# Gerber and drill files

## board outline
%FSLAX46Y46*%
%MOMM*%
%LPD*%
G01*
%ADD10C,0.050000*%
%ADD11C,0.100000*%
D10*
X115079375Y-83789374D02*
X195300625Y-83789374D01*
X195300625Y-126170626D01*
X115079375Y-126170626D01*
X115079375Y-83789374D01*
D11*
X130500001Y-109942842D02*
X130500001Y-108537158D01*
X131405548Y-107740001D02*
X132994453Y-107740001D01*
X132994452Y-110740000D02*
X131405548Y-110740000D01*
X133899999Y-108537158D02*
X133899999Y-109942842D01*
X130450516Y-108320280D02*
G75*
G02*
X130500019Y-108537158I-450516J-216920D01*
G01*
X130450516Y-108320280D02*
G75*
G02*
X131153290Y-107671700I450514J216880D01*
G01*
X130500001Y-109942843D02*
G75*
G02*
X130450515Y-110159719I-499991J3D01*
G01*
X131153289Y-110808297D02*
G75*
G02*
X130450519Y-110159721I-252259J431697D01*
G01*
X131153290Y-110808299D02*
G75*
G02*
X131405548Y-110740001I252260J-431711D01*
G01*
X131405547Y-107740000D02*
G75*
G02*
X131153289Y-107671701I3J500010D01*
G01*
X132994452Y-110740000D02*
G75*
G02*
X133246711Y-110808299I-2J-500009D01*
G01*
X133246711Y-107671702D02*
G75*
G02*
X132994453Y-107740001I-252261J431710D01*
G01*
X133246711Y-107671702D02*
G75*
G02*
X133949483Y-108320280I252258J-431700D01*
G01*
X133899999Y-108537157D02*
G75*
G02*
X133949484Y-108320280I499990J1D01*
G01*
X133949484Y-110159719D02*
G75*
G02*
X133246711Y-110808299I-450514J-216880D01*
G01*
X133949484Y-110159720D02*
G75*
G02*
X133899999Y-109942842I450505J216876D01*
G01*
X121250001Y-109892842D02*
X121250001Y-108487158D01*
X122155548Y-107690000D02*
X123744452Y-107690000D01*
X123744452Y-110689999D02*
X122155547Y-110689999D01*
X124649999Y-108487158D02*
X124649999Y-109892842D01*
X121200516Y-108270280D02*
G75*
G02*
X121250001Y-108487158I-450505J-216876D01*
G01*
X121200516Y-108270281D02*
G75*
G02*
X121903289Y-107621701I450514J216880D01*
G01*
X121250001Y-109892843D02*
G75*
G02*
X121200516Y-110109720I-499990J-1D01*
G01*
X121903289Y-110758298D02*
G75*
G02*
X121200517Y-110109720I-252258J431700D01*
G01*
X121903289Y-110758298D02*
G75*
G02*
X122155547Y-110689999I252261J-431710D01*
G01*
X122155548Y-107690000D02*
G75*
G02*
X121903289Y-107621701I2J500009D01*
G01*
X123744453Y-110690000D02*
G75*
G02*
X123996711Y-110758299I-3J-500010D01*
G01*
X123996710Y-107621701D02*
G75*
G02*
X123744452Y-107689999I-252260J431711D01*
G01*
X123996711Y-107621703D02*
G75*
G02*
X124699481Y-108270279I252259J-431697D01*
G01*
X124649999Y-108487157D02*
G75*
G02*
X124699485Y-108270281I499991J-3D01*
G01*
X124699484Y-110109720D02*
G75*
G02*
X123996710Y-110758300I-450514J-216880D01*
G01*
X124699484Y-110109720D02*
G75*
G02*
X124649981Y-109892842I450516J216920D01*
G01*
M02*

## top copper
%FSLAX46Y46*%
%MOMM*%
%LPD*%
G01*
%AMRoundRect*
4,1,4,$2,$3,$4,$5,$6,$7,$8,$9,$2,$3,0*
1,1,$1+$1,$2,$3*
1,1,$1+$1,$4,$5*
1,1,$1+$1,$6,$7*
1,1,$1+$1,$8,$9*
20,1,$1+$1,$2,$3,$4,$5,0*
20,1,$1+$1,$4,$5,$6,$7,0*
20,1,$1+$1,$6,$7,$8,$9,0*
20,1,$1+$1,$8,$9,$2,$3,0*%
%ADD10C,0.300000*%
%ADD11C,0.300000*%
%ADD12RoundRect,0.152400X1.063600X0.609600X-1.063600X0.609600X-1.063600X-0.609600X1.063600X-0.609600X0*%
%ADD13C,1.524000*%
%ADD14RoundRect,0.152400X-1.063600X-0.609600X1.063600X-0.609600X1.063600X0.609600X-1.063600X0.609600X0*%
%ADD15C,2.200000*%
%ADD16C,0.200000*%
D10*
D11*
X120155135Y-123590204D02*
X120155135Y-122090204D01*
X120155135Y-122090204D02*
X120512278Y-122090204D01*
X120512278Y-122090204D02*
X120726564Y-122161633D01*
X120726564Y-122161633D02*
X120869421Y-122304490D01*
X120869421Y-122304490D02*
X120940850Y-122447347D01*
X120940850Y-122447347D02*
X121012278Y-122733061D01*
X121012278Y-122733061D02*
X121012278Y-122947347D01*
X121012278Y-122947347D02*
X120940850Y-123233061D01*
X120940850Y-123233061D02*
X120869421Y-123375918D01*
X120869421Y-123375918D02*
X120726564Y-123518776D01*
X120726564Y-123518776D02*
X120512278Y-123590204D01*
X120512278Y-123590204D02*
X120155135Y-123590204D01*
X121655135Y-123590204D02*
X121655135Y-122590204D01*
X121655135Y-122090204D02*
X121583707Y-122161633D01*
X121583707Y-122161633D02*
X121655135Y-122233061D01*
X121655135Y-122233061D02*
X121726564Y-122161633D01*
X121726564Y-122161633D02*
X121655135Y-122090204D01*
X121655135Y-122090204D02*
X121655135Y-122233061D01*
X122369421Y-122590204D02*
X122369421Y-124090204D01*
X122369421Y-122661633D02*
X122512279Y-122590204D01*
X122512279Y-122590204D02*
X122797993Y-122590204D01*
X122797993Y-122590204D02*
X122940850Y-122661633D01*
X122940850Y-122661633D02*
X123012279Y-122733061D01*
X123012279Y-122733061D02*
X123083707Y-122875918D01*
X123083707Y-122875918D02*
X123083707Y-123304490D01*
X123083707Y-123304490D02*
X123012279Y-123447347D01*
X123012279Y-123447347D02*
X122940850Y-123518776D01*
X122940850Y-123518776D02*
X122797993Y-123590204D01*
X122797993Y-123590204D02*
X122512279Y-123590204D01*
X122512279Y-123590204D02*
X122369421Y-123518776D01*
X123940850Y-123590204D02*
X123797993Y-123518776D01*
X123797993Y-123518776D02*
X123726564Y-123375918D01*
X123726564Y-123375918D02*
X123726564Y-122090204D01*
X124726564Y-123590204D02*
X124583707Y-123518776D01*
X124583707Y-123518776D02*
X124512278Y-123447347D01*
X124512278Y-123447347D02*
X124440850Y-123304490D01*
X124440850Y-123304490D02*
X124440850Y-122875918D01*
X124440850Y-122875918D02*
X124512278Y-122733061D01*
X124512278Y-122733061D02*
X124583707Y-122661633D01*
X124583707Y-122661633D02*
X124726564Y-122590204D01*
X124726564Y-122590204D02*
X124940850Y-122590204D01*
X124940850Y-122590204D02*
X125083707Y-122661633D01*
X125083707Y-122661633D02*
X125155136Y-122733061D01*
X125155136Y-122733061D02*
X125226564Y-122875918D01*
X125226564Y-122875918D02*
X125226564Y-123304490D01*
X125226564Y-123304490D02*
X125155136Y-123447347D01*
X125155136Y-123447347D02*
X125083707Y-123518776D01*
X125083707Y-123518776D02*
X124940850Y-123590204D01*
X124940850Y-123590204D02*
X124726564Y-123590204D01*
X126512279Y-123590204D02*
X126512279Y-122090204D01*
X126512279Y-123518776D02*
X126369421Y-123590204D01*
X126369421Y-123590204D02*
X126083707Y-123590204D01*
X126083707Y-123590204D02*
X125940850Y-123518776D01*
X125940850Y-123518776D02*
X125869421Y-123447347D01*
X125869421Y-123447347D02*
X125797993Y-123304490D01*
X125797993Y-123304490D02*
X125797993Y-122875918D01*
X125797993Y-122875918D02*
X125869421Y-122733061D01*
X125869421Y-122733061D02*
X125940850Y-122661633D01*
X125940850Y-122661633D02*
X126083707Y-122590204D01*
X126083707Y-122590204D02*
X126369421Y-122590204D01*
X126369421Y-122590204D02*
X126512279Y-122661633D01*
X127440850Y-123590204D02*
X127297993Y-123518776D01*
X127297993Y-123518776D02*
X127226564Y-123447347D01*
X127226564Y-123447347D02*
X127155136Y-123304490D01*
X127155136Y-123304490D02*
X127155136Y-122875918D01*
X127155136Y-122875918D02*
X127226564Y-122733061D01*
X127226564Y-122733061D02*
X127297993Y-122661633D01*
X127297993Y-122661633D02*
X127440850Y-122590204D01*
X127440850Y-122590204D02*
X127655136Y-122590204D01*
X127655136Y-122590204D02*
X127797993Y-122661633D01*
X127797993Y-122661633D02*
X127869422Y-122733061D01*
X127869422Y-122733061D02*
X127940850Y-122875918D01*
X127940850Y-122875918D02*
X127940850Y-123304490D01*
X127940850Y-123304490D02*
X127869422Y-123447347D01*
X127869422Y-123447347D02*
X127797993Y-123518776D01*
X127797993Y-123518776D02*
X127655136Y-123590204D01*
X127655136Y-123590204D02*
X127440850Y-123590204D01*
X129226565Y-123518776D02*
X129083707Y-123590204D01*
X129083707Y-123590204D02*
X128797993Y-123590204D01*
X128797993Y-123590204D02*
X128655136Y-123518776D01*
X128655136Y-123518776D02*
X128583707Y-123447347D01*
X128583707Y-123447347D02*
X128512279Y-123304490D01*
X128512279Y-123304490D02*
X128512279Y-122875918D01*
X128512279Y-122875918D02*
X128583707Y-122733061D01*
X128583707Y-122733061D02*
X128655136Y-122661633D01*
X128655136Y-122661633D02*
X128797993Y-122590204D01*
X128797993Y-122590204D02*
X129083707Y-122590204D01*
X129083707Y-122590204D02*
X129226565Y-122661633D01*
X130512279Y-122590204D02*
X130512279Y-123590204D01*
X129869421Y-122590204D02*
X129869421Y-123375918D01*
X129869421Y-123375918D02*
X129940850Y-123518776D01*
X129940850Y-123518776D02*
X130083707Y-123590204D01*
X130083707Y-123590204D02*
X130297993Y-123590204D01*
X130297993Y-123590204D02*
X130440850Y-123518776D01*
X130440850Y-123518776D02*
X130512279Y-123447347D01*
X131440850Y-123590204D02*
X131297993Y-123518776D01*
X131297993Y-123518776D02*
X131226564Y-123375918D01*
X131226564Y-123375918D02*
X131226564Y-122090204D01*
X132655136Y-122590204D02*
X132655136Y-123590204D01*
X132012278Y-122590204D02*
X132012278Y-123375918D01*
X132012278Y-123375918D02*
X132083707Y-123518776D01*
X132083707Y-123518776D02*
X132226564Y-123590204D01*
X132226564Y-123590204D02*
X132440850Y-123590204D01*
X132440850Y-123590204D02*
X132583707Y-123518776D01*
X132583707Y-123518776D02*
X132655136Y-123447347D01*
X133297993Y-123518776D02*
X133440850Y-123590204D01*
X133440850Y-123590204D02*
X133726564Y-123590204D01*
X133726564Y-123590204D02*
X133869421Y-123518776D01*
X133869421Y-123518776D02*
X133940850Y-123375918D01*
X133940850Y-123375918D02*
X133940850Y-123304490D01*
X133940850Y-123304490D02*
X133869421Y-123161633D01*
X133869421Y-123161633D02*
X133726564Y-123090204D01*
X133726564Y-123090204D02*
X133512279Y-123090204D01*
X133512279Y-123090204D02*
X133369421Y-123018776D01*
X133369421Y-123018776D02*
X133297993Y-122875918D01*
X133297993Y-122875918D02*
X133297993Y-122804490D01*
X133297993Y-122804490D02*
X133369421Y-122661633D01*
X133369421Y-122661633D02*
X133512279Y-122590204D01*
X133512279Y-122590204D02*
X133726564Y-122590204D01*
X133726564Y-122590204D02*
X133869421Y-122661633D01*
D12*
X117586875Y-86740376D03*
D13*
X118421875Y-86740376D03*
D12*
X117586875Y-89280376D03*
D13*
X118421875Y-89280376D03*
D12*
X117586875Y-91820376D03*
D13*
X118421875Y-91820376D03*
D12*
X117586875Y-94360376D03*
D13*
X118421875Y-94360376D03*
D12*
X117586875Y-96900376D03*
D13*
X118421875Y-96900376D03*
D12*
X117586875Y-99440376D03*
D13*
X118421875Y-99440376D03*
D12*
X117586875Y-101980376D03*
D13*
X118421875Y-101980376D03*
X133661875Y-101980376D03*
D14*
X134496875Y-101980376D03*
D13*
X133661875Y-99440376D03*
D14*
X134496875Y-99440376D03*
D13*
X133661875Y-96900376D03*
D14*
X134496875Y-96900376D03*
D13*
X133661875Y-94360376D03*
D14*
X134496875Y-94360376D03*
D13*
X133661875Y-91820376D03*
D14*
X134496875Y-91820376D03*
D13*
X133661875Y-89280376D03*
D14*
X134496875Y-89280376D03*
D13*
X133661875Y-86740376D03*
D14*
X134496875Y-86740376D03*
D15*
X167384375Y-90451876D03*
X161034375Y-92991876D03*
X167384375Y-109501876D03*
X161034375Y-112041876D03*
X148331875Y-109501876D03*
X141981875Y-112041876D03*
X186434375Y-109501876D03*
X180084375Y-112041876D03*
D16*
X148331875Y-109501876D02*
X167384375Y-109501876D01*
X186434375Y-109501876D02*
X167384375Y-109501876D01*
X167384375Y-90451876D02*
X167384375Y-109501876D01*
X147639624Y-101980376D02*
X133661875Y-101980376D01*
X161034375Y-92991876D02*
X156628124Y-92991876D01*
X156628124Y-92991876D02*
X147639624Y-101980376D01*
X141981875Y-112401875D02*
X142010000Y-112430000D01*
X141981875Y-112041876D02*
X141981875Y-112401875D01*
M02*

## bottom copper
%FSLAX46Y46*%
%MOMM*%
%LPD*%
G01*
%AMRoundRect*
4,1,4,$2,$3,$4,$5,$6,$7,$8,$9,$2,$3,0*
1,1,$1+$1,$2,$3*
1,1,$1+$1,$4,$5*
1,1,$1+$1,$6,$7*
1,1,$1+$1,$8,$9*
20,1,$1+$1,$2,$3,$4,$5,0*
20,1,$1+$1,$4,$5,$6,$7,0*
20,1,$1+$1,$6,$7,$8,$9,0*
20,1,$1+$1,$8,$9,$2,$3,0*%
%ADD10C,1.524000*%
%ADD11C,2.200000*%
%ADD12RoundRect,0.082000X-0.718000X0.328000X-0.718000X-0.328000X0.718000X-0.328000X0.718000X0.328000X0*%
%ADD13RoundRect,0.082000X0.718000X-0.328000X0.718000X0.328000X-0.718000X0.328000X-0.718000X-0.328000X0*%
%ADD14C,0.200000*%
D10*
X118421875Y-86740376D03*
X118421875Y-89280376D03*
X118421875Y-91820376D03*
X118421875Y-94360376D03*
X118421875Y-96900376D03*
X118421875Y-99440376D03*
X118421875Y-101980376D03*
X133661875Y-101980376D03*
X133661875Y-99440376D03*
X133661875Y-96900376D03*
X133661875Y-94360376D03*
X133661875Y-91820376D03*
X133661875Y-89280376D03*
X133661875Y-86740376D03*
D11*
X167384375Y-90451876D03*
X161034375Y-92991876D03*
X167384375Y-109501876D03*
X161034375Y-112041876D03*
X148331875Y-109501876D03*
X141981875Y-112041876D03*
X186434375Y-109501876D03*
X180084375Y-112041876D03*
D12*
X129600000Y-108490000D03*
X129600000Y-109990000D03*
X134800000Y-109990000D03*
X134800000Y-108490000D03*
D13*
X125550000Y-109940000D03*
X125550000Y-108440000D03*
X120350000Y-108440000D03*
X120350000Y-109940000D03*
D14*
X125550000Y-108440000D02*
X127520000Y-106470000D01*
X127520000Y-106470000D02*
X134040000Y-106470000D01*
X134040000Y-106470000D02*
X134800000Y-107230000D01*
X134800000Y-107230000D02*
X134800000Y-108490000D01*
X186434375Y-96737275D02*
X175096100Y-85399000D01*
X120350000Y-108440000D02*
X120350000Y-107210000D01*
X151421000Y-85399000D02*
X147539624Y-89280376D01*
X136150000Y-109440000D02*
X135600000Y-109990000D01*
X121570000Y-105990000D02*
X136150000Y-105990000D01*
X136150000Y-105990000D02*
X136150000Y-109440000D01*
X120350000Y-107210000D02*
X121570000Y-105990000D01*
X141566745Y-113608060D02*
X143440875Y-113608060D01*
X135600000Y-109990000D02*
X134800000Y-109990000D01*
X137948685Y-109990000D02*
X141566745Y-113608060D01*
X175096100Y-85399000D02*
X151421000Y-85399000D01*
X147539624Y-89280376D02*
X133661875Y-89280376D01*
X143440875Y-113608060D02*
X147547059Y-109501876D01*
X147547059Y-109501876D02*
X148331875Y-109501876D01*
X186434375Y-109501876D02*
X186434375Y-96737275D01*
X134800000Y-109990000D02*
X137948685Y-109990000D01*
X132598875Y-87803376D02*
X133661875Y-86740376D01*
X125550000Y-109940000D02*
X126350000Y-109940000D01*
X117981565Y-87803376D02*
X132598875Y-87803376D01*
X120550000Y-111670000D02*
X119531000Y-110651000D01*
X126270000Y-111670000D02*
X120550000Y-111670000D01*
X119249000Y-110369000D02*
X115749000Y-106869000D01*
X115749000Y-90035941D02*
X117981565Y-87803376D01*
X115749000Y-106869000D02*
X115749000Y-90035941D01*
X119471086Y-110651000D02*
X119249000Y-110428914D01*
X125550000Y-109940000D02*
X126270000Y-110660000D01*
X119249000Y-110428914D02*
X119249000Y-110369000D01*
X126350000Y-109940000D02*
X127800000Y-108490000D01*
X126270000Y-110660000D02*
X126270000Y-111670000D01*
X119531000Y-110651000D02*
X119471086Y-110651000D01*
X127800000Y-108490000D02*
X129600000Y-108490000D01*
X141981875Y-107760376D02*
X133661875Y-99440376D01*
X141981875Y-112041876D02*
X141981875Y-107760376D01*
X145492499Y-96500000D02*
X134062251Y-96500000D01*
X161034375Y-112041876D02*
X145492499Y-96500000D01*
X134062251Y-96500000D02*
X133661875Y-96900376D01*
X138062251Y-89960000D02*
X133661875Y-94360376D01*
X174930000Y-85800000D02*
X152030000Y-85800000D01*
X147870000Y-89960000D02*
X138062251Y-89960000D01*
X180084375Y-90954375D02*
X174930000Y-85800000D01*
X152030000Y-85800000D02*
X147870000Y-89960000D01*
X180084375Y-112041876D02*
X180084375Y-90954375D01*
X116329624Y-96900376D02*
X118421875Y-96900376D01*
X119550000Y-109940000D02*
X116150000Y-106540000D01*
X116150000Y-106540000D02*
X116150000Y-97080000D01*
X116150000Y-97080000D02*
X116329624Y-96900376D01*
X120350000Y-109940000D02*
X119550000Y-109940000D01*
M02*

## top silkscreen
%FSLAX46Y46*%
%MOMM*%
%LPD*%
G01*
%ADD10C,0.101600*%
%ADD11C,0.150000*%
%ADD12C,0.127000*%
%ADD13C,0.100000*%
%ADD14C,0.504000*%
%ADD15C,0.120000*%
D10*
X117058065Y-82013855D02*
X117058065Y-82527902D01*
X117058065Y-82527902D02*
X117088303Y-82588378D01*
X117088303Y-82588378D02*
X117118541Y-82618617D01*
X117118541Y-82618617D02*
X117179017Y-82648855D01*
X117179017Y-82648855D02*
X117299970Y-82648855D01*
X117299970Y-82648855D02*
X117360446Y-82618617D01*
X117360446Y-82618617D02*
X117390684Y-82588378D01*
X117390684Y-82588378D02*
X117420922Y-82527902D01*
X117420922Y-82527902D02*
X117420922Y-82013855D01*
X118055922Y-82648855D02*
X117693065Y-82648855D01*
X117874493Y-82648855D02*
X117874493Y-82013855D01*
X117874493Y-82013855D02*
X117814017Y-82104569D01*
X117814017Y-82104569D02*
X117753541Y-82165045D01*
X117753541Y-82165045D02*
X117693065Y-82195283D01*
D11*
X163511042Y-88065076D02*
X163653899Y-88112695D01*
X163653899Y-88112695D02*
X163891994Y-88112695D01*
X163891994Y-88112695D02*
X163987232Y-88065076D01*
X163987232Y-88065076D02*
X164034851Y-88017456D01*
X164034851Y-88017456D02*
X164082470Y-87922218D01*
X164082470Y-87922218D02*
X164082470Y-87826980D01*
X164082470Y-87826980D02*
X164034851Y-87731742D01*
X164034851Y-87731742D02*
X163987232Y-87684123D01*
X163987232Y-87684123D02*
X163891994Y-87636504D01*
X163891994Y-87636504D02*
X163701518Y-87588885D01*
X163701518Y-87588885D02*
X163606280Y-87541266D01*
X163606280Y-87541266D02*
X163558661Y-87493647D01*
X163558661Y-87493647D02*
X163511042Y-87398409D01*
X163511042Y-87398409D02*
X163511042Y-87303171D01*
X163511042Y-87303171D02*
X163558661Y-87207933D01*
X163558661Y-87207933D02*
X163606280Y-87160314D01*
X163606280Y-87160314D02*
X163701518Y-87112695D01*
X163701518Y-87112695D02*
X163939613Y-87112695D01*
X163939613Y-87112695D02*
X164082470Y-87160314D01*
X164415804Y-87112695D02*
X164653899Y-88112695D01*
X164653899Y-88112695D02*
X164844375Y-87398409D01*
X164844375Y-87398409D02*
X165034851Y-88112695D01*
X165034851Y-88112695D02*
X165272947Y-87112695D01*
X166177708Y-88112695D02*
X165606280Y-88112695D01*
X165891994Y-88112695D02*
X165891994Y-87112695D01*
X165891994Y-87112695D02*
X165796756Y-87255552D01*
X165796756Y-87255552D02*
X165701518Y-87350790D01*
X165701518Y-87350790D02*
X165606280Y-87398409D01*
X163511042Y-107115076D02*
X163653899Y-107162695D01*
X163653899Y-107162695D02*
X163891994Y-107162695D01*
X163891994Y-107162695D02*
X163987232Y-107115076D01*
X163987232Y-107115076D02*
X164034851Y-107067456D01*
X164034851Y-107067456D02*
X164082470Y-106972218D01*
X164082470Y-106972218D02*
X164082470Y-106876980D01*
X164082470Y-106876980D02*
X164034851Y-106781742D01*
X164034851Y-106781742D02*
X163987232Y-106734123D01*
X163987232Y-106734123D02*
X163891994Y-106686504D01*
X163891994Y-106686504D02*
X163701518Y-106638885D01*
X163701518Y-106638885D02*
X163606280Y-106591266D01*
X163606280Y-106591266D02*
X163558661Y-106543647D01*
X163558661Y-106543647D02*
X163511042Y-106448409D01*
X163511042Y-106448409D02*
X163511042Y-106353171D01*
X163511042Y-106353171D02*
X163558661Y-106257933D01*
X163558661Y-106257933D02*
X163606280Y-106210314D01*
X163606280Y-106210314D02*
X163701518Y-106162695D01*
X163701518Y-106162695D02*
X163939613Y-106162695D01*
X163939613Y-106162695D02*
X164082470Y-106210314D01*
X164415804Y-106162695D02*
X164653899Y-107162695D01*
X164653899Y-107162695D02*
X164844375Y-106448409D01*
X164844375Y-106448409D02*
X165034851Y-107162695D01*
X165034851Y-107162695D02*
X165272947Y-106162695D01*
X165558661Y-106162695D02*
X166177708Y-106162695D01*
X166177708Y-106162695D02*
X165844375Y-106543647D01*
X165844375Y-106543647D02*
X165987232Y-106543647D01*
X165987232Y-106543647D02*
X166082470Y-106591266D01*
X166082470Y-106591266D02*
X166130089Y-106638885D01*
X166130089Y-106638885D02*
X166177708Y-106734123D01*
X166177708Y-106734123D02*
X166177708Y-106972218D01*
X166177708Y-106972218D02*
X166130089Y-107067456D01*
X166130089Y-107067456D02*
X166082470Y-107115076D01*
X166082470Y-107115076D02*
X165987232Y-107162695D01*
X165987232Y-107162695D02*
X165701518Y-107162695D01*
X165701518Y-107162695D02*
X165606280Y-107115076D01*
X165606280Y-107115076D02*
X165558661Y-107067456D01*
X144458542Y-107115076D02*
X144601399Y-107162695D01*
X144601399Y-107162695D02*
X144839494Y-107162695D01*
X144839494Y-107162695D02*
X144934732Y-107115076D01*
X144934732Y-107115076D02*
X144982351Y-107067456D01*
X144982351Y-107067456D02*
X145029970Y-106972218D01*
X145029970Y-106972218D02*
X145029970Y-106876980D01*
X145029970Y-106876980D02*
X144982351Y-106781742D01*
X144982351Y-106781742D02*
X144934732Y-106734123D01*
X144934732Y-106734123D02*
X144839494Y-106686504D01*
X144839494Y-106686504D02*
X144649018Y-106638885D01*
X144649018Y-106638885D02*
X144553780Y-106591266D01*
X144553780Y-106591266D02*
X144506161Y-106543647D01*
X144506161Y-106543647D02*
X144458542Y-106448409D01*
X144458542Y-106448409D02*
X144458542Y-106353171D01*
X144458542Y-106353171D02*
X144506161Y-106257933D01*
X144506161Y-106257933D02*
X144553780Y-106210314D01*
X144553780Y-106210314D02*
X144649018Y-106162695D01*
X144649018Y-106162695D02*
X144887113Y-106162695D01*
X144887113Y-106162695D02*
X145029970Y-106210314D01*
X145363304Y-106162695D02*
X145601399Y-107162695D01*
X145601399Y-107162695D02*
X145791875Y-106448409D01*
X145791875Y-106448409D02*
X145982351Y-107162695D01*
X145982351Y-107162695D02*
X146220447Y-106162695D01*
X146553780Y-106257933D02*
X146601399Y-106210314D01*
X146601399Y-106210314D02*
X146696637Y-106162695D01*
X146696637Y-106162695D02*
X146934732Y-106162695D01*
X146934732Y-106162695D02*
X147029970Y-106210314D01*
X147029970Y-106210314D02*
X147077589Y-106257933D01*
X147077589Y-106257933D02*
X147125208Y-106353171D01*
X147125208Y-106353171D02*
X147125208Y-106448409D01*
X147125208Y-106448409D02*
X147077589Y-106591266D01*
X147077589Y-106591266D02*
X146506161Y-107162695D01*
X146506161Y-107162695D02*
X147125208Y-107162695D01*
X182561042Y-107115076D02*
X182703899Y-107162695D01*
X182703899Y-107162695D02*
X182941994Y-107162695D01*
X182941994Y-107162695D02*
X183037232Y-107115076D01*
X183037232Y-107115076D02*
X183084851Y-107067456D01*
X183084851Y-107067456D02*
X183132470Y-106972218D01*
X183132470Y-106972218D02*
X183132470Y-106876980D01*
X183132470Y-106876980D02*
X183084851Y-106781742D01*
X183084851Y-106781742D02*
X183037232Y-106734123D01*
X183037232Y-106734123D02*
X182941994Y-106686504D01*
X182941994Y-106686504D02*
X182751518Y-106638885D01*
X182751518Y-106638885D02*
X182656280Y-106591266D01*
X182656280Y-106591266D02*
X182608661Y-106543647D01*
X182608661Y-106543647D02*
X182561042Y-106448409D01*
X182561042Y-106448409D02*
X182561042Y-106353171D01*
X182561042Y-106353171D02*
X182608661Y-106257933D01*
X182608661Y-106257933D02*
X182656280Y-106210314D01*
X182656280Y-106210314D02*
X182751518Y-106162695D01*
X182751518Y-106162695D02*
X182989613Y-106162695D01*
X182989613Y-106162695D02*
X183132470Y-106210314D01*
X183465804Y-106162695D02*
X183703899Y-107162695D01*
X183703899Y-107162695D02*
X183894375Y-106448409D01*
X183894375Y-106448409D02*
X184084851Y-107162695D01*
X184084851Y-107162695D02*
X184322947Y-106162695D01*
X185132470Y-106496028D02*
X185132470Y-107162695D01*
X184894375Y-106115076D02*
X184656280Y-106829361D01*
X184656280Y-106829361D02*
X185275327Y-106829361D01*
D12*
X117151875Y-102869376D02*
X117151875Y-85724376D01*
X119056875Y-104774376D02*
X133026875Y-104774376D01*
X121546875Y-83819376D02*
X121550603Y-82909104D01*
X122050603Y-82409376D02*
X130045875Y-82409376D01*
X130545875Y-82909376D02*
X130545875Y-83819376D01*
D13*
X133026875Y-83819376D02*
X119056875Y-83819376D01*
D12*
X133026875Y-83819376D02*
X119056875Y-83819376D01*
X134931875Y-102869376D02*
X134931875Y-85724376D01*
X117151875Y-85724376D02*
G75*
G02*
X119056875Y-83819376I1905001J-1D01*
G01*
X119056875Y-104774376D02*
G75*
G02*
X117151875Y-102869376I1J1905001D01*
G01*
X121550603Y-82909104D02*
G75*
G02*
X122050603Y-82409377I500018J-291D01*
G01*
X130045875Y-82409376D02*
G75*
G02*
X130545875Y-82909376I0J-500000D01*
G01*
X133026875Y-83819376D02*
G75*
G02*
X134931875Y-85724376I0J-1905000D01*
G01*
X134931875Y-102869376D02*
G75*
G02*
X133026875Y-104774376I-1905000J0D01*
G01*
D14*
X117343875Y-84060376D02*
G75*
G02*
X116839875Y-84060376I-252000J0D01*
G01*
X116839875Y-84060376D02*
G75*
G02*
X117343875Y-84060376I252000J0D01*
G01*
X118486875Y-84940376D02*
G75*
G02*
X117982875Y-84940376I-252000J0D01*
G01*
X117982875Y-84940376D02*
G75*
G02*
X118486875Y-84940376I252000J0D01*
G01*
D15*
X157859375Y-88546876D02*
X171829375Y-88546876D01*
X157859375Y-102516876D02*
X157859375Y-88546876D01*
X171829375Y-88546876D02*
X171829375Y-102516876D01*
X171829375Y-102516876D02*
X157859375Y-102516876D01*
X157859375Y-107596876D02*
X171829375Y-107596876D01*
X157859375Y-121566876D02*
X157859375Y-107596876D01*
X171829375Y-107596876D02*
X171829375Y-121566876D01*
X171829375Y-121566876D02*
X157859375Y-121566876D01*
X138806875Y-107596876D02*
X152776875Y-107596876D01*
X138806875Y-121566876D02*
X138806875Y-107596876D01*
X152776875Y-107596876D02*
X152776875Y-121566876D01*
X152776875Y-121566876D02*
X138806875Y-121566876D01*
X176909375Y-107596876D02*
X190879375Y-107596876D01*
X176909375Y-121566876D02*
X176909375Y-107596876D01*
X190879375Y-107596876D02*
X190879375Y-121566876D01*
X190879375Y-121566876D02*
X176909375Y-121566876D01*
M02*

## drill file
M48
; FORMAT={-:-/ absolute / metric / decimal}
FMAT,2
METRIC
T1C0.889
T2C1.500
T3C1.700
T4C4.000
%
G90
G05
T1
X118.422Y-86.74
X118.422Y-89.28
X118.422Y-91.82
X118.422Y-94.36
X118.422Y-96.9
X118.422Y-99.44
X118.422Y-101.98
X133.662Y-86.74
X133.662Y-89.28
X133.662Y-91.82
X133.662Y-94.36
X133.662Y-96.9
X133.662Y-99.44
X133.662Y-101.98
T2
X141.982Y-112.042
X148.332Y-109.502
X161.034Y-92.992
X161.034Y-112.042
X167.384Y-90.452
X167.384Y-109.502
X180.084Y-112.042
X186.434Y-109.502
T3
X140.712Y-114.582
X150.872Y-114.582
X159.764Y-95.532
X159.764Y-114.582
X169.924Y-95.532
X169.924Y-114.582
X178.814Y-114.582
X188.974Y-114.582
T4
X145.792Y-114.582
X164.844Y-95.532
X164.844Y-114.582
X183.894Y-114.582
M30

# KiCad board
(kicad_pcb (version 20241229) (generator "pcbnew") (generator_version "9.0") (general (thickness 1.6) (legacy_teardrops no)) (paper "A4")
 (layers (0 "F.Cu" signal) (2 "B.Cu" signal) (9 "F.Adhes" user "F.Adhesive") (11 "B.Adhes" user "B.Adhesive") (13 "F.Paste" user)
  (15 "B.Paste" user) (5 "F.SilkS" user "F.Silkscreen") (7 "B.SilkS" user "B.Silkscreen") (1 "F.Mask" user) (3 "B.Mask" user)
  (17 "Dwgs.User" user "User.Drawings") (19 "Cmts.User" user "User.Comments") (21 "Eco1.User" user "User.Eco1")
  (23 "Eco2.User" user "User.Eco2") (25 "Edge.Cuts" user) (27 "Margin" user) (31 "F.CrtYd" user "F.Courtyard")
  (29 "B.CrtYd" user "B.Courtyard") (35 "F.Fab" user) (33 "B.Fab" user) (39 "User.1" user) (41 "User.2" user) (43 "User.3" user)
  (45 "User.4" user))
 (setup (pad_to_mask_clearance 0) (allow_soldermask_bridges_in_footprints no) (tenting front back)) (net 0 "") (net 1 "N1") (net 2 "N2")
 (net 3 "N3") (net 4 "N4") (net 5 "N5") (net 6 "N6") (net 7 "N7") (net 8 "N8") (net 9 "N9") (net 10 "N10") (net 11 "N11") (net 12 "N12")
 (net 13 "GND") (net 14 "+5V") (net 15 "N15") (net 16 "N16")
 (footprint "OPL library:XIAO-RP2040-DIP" (layer "F.Cu") (at 126.041875 94.360376)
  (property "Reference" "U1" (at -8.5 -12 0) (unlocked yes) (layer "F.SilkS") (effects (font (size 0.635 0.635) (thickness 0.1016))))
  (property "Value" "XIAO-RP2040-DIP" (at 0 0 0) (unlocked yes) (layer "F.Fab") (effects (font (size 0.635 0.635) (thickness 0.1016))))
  (fp_line (start -8.89 8.509) (end -8.89 -8.636) (stroke (width 0.127) (type solid)) (layer "F.SilkS"))
  (fp_line (start -6.985 10.414) (end 6.985 10.414) (stroke (width 0.127) (type solid)) (layer "F.SilkS"))
  (fp_line (start -4.495 -10.541) (end -4.491272 -11.451272) (stroke (width 0.127) (type solid)) (layer "F.SilkS"))
  (fp_line (start -3.991272 -11.951) (end 4.004 -11.951) (stroke (width 0.127) (type solid)) (layer "F.SilkS"))
  (fp_line (start 4.504 -11.451) (end 4.504 -10.541) (stroke (width 0.127) (type solid)) (layer "F.SilkS"))
  (fp_line (start 6.985 -10.541) (end -6.985 -10.541) (stroke (width 0.1) (type solid)) (layer "F.SilkS"))
  (fp_line (start 6.985 -10.541) (end -6.985 -10.541) (stroke (width 0.127) (type solid)) (layer "F.SilkS"))
  (fp_line (start 8.89 8.509) (end 8.89 -8.636) (stroke (width 0.127) (type solid)) (layer "F.SilkS"))
  (fp_arc (start -8.89 -8.636) (mid -8.332038 -9.983038) (end -6.985 -10.541) (stroke (width 0.127) (type solid)) (layer "F.SilkS"))
  (fp_arc (start -6.985 10.414) (mid -8.332038 9.856038) (end -8.89 8.509) (stroke (width 0.127) (type solid)) (layer "F.SilkS"))
  (fp_arc (start -4.491272 -11.451272) (mid -4.344728 -11.80464) (end -3.991272 -11.951) (stroke (width 0.127) (type default))
   (layer "F.SilkS"))
  (fp_arc (start 4.004 -11.951) (mid 4.357553 -11.804553) (end 4.504 -11.451) (stroke (width 0.127) (type default)) (layer "F.SilkS"))
  (fp_arc (start 6.985 -10.541) (mid 8.332038 -9.983038) (end 8.89 -8.636) (stroke (width 0.127) (type solid)) (layer "F.SilkS"))
  (fp_arc (start 8.89 8.509) (mid 8.332038 9.856038) (end 6.985 10.414) (stroke (width 0.127) (type solid)) (layer "F.SilkS"))
  (fp_circle (center -8.95 -10.3) (end -8.95 -10.554) (stroke (width 0.5) (type solid)) (fill yes) (layer "F.SilkS"))
  (fp_circle (center -7.807 -9.42) (end -7.807 -9.674) (stroke (width 0.5) (type solid)) (fill yes) (layer "F.SilkS"))
  (pad "1" smd roundrect (at -8.455 -7.62 180) (size 2.432 1.524) (layers "F.Cu" "F.Mask") (roundrect_rratio 0.1) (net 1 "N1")
   (thermal_bridge_angle 45))
  (pad "1" thru_hole circle (at -7.62 -7.62 180) (size 1.524 1.524) (drill 0.889) (layers "*.Cu" "*.Mask") (remove_unused_layers no)
   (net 1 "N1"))
  (pad "2" smd roundrect (at -8.455 -5.08 180) (size 2.432 1.524) (layers "F.Cu" "F.Mask") (roundrect_rratio 0.1) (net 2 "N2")
   (thermal_bridge_angle 45))
  (pad "2" thru_hole circle (at -7.62 -5.08 180) (size 1.524 1.524) (drill 0.889) (layers "*.Cu" "*.Mask") (remove_unused_layers no)
   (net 2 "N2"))
  (pad "3" smd roundrect (at -8.455 -2.54 180) (size 2.432 1.524) (layers "F.Cu" "F.Mask") (roundrect_rratio 0.1) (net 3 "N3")
   (thermal_bridge_angle 45))
  (pad "3" thru_hole circle (at -7.62 -2.54 180) (size 1.524 1.524) (drill 0.889) (layers "*.Cu" "*.Mask") (remove_unused_layers no)
   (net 3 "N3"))
  (pad "4" smd roundrect (at -8.455 0 180) (size 2.432 1.524) (layers "F.Cu" "F.Mask") (roundrect_rratio 0.1) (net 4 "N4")
   (thermal_bridge_angle 45))
  (pad "4" thru_hole circle (at -7.62 0 180) (size 1.524 1.524) (drill 0.889) (layers "*.Cu" "*.Mask") (remove_unused_layers no)
   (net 4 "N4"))
  (pad "5" smd roundrect (at -8.455 2.54 180) (size 2.432 1.524) (layers "F.Cu" "F.Mask") (roundrect_rratio 0.1) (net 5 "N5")
   (thermal_bridge_angle 45))
  (pad "5" thru_hole circle (at -7.62 2.54 180) (size 1.524 1.524) (drill 0.889) (layers "*.Cu" "*.Mask") (remove_unused_layers no)
   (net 5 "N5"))
  (pad "6" smd roundrect (at -8.455 5.08 180) (size 2.432 1.524) (layers "F.Cu" "F.Mask") (roundrect_rratio 0.1) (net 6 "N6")
   (thermal_bridge_angle 45))
  (pad "6" thru_hole circle (at -7.62 5.08 180) (size 1.524 1.524) (drill 0.889) (layers "*.Cu" "*.Mask") (remove_unused_layers no)
   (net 6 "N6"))
  (pad "7" smd roundrect (at -8.455 7.62 180) (size 2.432 1.524) (layers "F.Cu" "F.Mask") (roundrect_rratio 0.1) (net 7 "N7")
   (thermal_bridge_angle 45))
  (pad "7" thru_hole circle (at -7.62 7.62 180) (size 1.524 1.524) (drill 0.889) (layers "*.Cu" "*.Mask") (remove_unused_layers no)
   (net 7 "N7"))
  (pad "8" thru_hole circle (at 7.62 7.62) (size 1.524 1.524) (drill 0.889) (layers "*.Cu" "*.Mask") (remove_unused_layers no) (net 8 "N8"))
  (pad "8" smd roundrect (at 8.455 7.62) (size 2.432 1.524) (layers "F.Cu" "F.Mask") (roundrect_rratio 0.1) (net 8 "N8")
   (thermal_bridge_angle 45))
  (pad "9" thru_hole circle (at 7.62 5.08) (size 1.524 1.524) (drill 0.889) (layers "*.Cu" "*.Mask") (remove_unused_layers no) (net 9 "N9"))
  (pad "9" smd roundrect (at 8.455 5.08) (size 2.432 1.524) (layers "F.Cu" "F.Mask") (roundrect_rratio 0.1) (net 9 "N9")
   (thermal_bridge_angle 45))
  (pad "10" thru_hole circle (at 7.62 2.54) (size 1.524 1.524) (drill 0.889) (layers "*.Cu" "*.Mask") (remove_unused_layers no)
   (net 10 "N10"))
  (pad "10" smd roundrect (at 8.455 2.54) (size 2.432 1.524) (layers "F.Cu" "F.Mask") (roundrect_rratio 0.1) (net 10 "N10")
   (thermal_bridge_angle 45))
  (pad "11" thru_hole circle (at 7.62 0) (size 1.524 1.524) (drill 0.889) (layers "*.Cu" "*.Mask") (remove_unused_layers no) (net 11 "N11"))
  (pad "11" smd roundrect (at 8.455 0) (size 2.432 1.524) (layers "F.Cu" "F.Mask") (roundrect_rratio 0.1) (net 11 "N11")
   (thermal_bridge_angle 45))
  (pad "12" thru_hole circle (at 7.62 -2.54) (size 1.524 1.524) (drill 0.889) (layers "*.Cu" "*.Mask") (remove_unused_layers no)
   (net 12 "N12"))
  (pad "12" smd roundrect (at 8.455 -2.54) (size 2.432 1.524) (layers "F.Cu" "F.Mask") (roundrect_rratio 0.1) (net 12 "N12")
   (thermal_bridge_angle 45))
  (pad "13" thru_hole circle (at 7.62 -5.08) (size 1.524 1.524) (drill 0.889) (layers "*.Cu" "*.Mask") (remove_unused_layers no)
   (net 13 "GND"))
  (pad "13" smd roundrect (at 8.455 -5.08) (size 2.432 1.524) (layers "F.Cu" "F.Mask") (roundrect_rratio 0.1) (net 13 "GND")
   (thermal_bridge_angle 45))
  (pad "14" thru_hole circle (at 7.62 -7.62) (size 1.524 1.524) (drill 0.889) (layers "*.Cu" "*.Mask") (remove_unused_layers no)
   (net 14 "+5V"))
  (pad "14" smd roundrect (at 8.455 -7.62) (size 2.432 1.524) (layers "F.Cu" "F.Mask") (roundrect_rratio 0.1) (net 14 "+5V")
   (thermal_bridge_angle 45)))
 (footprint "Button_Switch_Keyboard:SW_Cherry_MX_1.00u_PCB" (layer "F.Cu") (at 167.384375 90.451876)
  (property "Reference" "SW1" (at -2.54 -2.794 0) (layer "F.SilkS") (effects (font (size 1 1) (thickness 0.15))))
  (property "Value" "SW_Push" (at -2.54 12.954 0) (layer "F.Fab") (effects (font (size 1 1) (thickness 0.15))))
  (fp_line (start -9.525 -1.905) (end 4.445 -1.905) (stroke (width 0.12) (type solid)) (layer "F.SilkS"))
  (fp_line (start -9.525 12.065) (end -9.525 -1.905) (stroke (width 0.12) (type solid)) (layer "F.SilkS"))
  (fp_line (start 4.445 -1.905) (end 4.445 12.065) (stroke (width 0.12) (type solid)) (layer "F.SilkS"))
  (fp_line (start 4.445 12.065) (end -9.525 12.065) (stroke (width 0.12) (type solid)) (layer "F.SilkS"))
  (pad "" np_thru_hole circle (at -7.62 5.08) (size 1.7 1.7) (drill 1.7) (layers "*.Cu" "*.Mask"))
  (pad "" np_thru_hole circle (at -2.54 5.08) (size 4 4) (drill 4) (layers "*.Cu" "*.Mask"))
  (pad "" np_thru_hole circle (at 2.54 5.08) (size 1.7 1.7) (drill 1.7) (layers "*.Cu" "*.Mask"))
  (pad "1" thru_hole circle (at 0 0) (size 2.2 2.2) (drill 1.5) (layers "*.Cu" "*.Mask") (remove_unused_layers no) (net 13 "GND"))
  (pad "2" thru_hole circle (at -6.35 2.54) (size 2.2 2.2) (drill 1.5) (layers "*.Cu" "*.Mask") (remove_unused_layers no) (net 8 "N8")))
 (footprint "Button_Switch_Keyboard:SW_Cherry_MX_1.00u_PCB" (layer "F.Cu") (at 167.384375 109.501876)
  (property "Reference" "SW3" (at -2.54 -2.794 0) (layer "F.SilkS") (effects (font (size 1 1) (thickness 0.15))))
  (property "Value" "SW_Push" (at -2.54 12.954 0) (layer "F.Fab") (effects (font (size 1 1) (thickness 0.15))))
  (fp_line (start -9.525 -1.905) (end 4.445 -1.905) (stroke (width 0.12) (type solid)) (layer "F.SilkS"))
  (fp_line (start -9.525 12.065) (end -9.525 -1.905) (stroke (width 0.12) (type solid)) (layer "F.SilkS"))
  (fp_line (start 4.445 -1.905) (end 4.445 12.065) (stroke (width 0.12) (type solid)) (layer "F.SilkS"))
  (fp_line (start 4.445 12.065) (end -9.525 12.065) (stroke (width 0.12) (type solid)) (layer "F.SilkS"))
  (pad "" np_thru_hole circle (at -7.62 5.08) (size 1.7 1.7) (drill 1.7) (layers "*.Cu" "*.Mask"))
  (pad "" np_thru_hole circle (at -2.54 5.08) (size 4 4) (drill 4) (layers "*.Cu" "*.Mask"))
  (pad "" np_thru_hole circle (at 2.54 5.08) (size 1.7 1.7) (drill 1.7) (layers "*.Cu" "*.Mask"))
  (pad "1" thru_hole circle (at 0 0) (size 2.2 2.2) (drill 1.5) (layers "*.Cu" "*.Mask") (remove_unused_layers no) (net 13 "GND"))
  (pad "2" thru_hole circle (at -6.35 2.54) (size 2.2 2.2) (drill 1.5) (layers "*.Cu" "*.Mask") (remove_unused_layers no) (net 10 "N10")))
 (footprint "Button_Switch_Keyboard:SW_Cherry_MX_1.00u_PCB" (layer "F.Cu") (at 148.331875 109.501876)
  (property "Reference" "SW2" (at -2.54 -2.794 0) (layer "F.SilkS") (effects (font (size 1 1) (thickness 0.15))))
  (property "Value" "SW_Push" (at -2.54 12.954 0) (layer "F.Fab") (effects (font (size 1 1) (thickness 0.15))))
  (fp_line (start -9.525 -1.905) (end 4.445 -1.905) (stroke (width 0.12) (type solid)) (layer "F.SilkS"))
  (fp_line (start -9.525 12.065) (end -9.525 -1.905) (stroke (width 0.12) (type solid)) (layer "F.SilkS"))
  (fp_line (start 4.445 -1.905) (end 4.445 12.065) (stroke (width 0.12) (type solid)) (layer "F.SilkS"))
  (fp_line (start 4.445 12.065) (end -9.525 12.065) (stroke (width 0.12) (type solid)) (layer "F.SilkS"))
  (pad "" np_thru_hole circle (at -7.62 5.08) (size 1.7 1.7) (drill 1.7) (layers "*.Cu" "*.Mask"))
  (pad "" np_thru_hole circle (at -2.54 5.08) (size 4 4) (drill 4) (layers "*.Cu" "*.Mask"))
  (pad "" np_thru_hole circle (at 2.54 5.08) (size 1.7 1.7) (drill 1.7) (layers "*.Cu" "*.Mask"))
  (pad "1" thru_hole circle (at 0 0) (size 2.2 2.2) (drill 1.5) (layers "*.Cu" "*.Mask") (remove_unused_layers no) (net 13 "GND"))
  (pad "2" thru_hole circle (at -6.35 2.54) (size 2.2 2.2) (drill 1.5) (layers "*.Cu" "*.Mask") (remove_unused_layers no) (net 9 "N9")))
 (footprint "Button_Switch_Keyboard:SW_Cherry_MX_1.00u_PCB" (layer "F.Cu") (at 186.434375 109.501876)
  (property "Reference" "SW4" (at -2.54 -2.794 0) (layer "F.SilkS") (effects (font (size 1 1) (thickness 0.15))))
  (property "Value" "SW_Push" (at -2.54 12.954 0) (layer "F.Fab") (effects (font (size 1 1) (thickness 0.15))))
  (fp_line (start -9.525 -1.905) (end 4.445 -1.905) (stroke (width 0.12) (type solid)) (layer "F.SilkS"))
  (fp_line (start -9.525 12.065) (end -9.525 -1.905) (stroke (width 0.12) (type solid)) (layer "F.SilkS"))
  (fp_line (start 4.445 -1.905) (end 4.445 12.065) (stroke (width 0.12) (type solid)) (layer "F.SilkS"))
  (fp_line (start 4.445 12.065) (end -9.525 12.065) (stroke (width 0.12) (type solid)) (layer "F.SilkS"))
  (pad "" np_thru_hole circle (at -7.62 5.08) (size 1.7 1.7) (drill 1.7) (layers "*.Cu" "*.Mask"))
  (pad "" np_thru_hole circle (at -2.54 5.08) (size 4 4) (drill 4) (layers "*.Cu" "*.Mask"))
  (pad "" np_thru_hole circle (at 2.54 5.08) (size 1.7 1.7) (drill 1.7) (layers "*.Cu" "*.Mask"))
  (pad "1" thru_hole circle (at 0 0) (size 2.2 2.2) (drill 1.5) (layers "*.Cu" "*.Mask") (remove_unused_layers no) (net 13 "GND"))
  (pad "2" thru_hole circle (at -6.35 2.54) (size 2.2 2.2) (drill 1.5) (layers "*.Cu" "*.Mask") (remove_unused_layers no) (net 11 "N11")))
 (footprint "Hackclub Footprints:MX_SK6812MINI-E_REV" (layer "F.Cu") (at 132.2 114.32 180)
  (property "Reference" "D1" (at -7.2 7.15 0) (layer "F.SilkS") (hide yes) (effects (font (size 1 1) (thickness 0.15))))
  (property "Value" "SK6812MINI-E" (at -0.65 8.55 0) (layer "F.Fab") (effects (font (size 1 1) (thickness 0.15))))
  (fp_line (start 1.699999 4.377158) (end 1.699999 5.782842) (stroke (width 0.1) (type solid)) (layer "Edge.Cuts"))
  (fp_line (start 0.794452 6.579999) (end -0.794453 6.579999) (stroke (width 0.1) (type solid)) (layer "Edge.Cuts"))
  (fp_line (start -0.794452 3.58) (end 0.794452 3.58) (stroke (width 0.1) (type solid)) (layer "Edge.Cuts"))
  (fp_line (start -1.699999 5.782842) (end -1.699999 4.377158) (stroke (width 0.1) (type solid)) (layer "Edge.Cuts"))
  (fp_arc (start 1.749484 5.99972) (mid 1.712527 5.894068) (end 1.699999 5.782842) (stroke (width 0.1) (type solid)) (layer "Edge.Cuts"))
  (fp_arc (start 1.749484 5.99972) (mid 1.638071 6.584035) (end 1.046711 6.648299) (stroke (width 0.1) (type solid)) (layer "Edge.Cuts"))
  (fp_arc (start 1.699999 4.377157) (mid 1.712527 4.265932) (end 1.749484 4.16028) (stroke (width 0.1) (type solid)) (layer "Edge.Cuts"))
  (fp_arc (start 1.046711 3.511703) (mid 1.63807 3.575966) (end 1.749484 4.16028) (stroke (width 0.1) (type solid)) (layer "Edge.Cuts"))
  (fp_arc (start 1.04671 3.511701) (mid 0.925122 3.562623) (end 0.794452 3.58) (stroke (width 0.1) (type solid)) (layer "Edge.Cuts"))
  (fp_arc (start 0.794453 6.58) (mid 0.925123 6.597377) (end 1.046711 6.648299) (stroke (width 0.1) (type solid)) (layer "Edge.Cuts"))
  (fp_arc (start -0.794452 3.58) (mid -0.925123 3.562623) (end -1.046711 3.511701) (stroke (width 0.1) (type solid)) (layer "Edge.Cuts"))
  (fp_arc (start -1.046711 6.648298) (mid -0.925123 6.597376) (end -0.794453 6.579999) (stroke (width 0.1) (type solid)) (layer "Edge.Cuts"))
  (fp_arc (start -1.046711 6.648298) (mid -1.638071 6.584034) (end -1.749484 5.99972) (stroke (width 0.1) (type solid)) (layer "Edge.Cuts"))
  (fp_arc (start -1.699999 5.782843) (mid -1.712527 5.894068) (end -1.749484 5.99972) (stroke (width 0.1) (type solid)) (layer "Edge.Cuts"))
  (fp_arc (start -1.749484 4.160281) (mid -1.638072 3.575965) (end -1.046711 3.511701) (stroke (width 0.1) (type solid)) (layer "Edge.Cuts"))
  (fp_arc (start -1.749484 4.16028) (mid -1.712527 4.265932) (end -1.699999 4.377158) (stroke (width 0.1) (type solid)) (layer "Edge.Cuts"))
  (pad "1" smd roundrect (at 2.6 5.83 270) (size 0.82 1.6) (layers "B.Cu" "B.Mask" "B.Paste") (roundrect_rratio 0.1) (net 14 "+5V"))
  (pad "2" smd roundrect (at 2.6 4.33 270) (size 0.82 1.6) (layers "B.Cu" "B.Mask" "B.Paste") (roundrect_rratio 0.1) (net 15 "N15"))
  (pad "3" smd roundrect (at -2.6 4.33 270) (size 0.82 1.6) (layers "B.Cu" "B.Mask" "B.Paste") (roundrect_rratio 0.1) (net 13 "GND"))
  (pad "4" smd roundrect (at -2.6 5.83 270) (size 0.82 1.6) (layers "B.Cu" "B.Mask" "B.Paste") (roundrect_rratio 0.1) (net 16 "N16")))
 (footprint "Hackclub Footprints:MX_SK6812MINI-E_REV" (layer "F.Cu") (at 122.95 104.11)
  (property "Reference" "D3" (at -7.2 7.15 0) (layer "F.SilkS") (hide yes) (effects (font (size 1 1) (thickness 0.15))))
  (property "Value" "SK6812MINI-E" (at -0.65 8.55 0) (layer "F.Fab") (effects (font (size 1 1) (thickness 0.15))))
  (fp_line (start -1.699999 5.782842) (end -1.699999 4.377158) (stroke (width 0.1) (type solid)) (layer "Edge.Cuts"))
  (fp_line (start -0.794452 3.58) (end 0.794452 3.58) (stroke (width 0.1) (type solid)) (layer "Edge.Cuts"))
  (fp_line (start 0.794452 6.579999) (end -0.794453 6.579999) (stroke (width 0.1) (type solid)) (layer "Edge.Cuts"))
  (fp_line (start 1.699999 4.377158) (end 1.699999 5.782842) (stroke (width 0.1) (type solid)) (layer "Edge.Cuts"))
  (fp_arc (start -1.749484 4.16028) (mid -1.712527 4.265932) (end -1.699999 4.377158) (stroke (width 0.1) (type solid)) (layer "Edge.Cuts"))
  (fp_arc (start -1.749484 4.160281) (mid -1.638072 3.575965) (end -1.046711 3.511701) (stroke (width 0.1) (type solid)) (layer "Edge.Cuts"))
  (fp_arc (start -1.699999 5.782843) (mid -1.712527 5.894068) (end -1.749484 5.99972) (stroke (width 0.1) (type solid)) (layer "Edge.Cuts"))
  (fp_arc (start -1.046711 6.648298) (mid -1.638071 6.584034) (end -1.749484 5.99972) (stroke (width 0.1) (type solid)) (layer "Edge.Cuts"))
  (fp_arc (start -1.046711 6.648298) (mid -0.925123 6.597376) (end -0.794453 6.579999) (stroke (width 0.1) (type solid)) (layer "Edge.Cuts"))
  (fp_arc (start -0.794452 3.58) (mid -0.925123 3.562623) (end -1.046711 3.511701) (stroke (width 0.1) (type solid)) (layer "Edge.Cuts"))
  (fp_arc (start 0.794453 6.58) (mid 0.925123 6.597377) (end 1.046711 6.648299) (stroke (width 0.1) (type solid)) (layer "Edge.Cuts"))
  (fp_arc (start 1.04671 3.511701) (mid 0.925122 3.562623) (end 0.794452 3.58) (stroke (width 0.1) (type solid)) (layer "Edge.Cuts"))
  (fp_arc (start 1.046711 3.511703) (mid 1.63807 3.575966) (end 1.749484 4.16028) (stroke (width 0.1) (type solid)) (layer "Edge.Cuts"))
  (fp_arc (start 1.699999 4.377157) (mid 1.712527 4.265932) (end 1.749484 4.16028) (stroke (width 0.1) (type solid)) (layer "Edge.Cuts"))
  (fp_arc (start 1.749484 5.99972) (mid 1.638071 6.584035) (end 1.046711 6.648299) (stroke (width 0.1) (type solid)) (layer "Edge.Cuts"))
  (fp_arc (start 1.749484 5.99972) (mid 1.712527 5.894068) (end 1.699999 5.782842) (stroke (width 0.1) (type solid)) (layer "Edge.Cuts"))
  (pad "1" smd roundrect (at 2.6 5.83 90) (size 0.82 1.6) (layers "B.Cu" "B.Mask" "B.Paste") (roundrect_rratio 0.1) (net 14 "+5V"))
  (pad "2" smd roundrect (at 2.6 4.33 90) (size 0.82 1.6) (layers "B.Cu" "B.Mask" "B.Paste") (roundrect_rratio 0.1) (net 16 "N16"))
  (pad "3" smd roundrect (at -2.6 4.33 90) (size 0.82 1.6) (layers "B.Cu" "B.Mask" "B.Paste") (roundrect_rratio 0.1) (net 13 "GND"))
  (pad "4" smd roundrect (at -2.6 5.83 90) (size 0.82 1.6) (layers "B.Cu" "B.Mask" "B.Paste") (roundrect_rratio 0.1) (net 5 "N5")))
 (gr_rect (start 115.079375 83.789374) (end 195.300625 126.170626) (stroke (width 0.05) (type default)) (fill no) (layer "Edge.Cuts"))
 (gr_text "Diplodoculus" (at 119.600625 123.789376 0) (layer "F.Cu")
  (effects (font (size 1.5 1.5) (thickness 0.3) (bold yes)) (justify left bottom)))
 (segment (start 125.55 108.44) (end 127.52 106.47) (width 0.2) (layer "B.Cu") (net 16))
 (segment (start 127.52 106.47) (end 134.04 106.47) (width 0.2) (layer "B.Cu") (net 16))
 (segment (start 134.04 106.47) (end 134.8 107.23) (width 0.2) (layer "B.Cu") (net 16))
 (segment (start 134.8 107.23) (end 134.8 108.49) (width 0.2) (layer "B.Cu") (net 16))
 (segment (start 148.331875 109.501876) (end 167.384375 109.501876) (width 0.2) (layer "F.Cu") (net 13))
 (segment (start 186.434375 109.501876) (end 167.384375 109.501876) (width 0.2) (layer "F.Cu") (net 13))
 (segment (start 167.384375 90.451876) (end 167.384375 109.501876) (width 0.2) (layer "F.Cu") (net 13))
 (segment (start 186.434375 96.737275) (end 175.0961 85.399) (width 0.2) (layer "B.Cu") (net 13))
 (segment (start 120.35 108.44) (end 120.35 107.21) (width 0.2) (layer "B.Cu") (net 13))
 (segment (start 151.421 85.399) (end 147.539624 89.280376) (width 0.2) (layer "B.Cu") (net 13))
 (segment (start 136.15 109.44) (end 135.6 109.99) (width 0.2) (layer "B.Cu") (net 13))
 (segment (start 121.57 105.99) (end 136.15 105.99) (width 0.2) (layer "B.Cu") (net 13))
 (segment (start 136.15 105.99) (end 136.15 109.44) (width 0.2) (layer "B.Cu") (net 13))
 (segment (start 120.35 107.21) (end 121.57 105.99) (width 0.2) (layer "B.Cu") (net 13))
 (segment (start 141.566745 113.60806) (end 143.440875 113.60806) (width 0.2) (layer "B.Cu") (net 13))
 (segment (start 135.6 109.99) (end 134.8 109.99) (width 0.2) (layer "B.Cu") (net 13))
 (segment (start 137.948685 109.99) (end 141.566745 113.60806) (width 0.2) (layer "B.Cu") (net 13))
 (segment (start 175.0961 85.399) (end 151.421 85.399) (width 0.2) (layer "B.Cu") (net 13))
 (segment (start 147.539624 89.280376) (end 133.661875 89.280376) (width 0.2) (layer "B.Cu") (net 13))
 (segment (start 143.440875 113.60806) (end 147.547059 109.501876) (width 0.2) (layer "B.Cu") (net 13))
 (segment (start 147.547059 109.501876) (end 148.331875 109.501876) (width 0.2) (layer "B.Cu") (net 13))
 (segment (start 186.434375 109.501876) (end 186.434375 96.737275) (width 0.2) (layer "B.Cu") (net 13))
 (segment (start 134.8 109.99) (end 137.948685 109.99) (width 0.2) (layer "B.Cu") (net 13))
 (segment (start 132.598875 87.803376) (end 133.661875 86.740376) (width 0.2) (layer "B.Cu") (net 14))
 (segment (start 125.55 109.94) (end 126.35 109.94) (width 0.2) (layer "B.Cu") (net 14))
 (segment (start 117.981565 87.803376) (end 132.598875 87.803376) (width 0.2) (layer "B.Cu") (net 14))
 (segment (start 120.55 111.67) (end 119.531 110.651) (width 0.2) (layer "B.Cu") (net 14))
 (segment (start 126.27 111.67) (end 120.55 111.67) (width 0.2) (layer "B.Cu") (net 14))
 (segment (start 119.249 110.369) (end 115.749 106.869) (width 0.2) (layer "B.Cu") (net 14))
 (segment (start 115.749 90.035941) (end 117.981565 87.803376) (width 0.2) (layer "B.Cu") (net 14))
 (segment (start 115.749 106.869) (end 115.749 90.035941) (width 0.2) (layer "B.Cu") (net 14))
 (segment (start 119.471086 110.651) (end 119.249 110.428914) (width 0.2) (layer "B.Cu") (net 14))
 (segment (start 125.55 109.94) (end 126.27 110.66) (width 0.2) (layer "B.Cu") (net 14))
 (segment (start 119.249 110.428914) (end 119.249 110.369) (width 0.2) (layer "B.Cu") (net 14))
 (segment (start 126.35 109.94) (end 127.8 108.49) (width 0.2) (layer "B.Cu") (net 14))
 (segment (start 126.27 110.66) (end 126.27 111.67) (width 0.2) (layer "B.Cu") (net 14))
 (segment (start 119.531 110.651) (end 119.471086 110.651) (width 0.2) (layer "B.Cu") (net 14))
 (segment (start 127.8 108.49) (end 129.6 108.49) (width 0.2) (layer "B.Cu") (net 14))
 (segment (start 147.639624 101.980376) (end 133.661875 101.980376) (width 0.2) (layer "F.Cu") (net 8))
 (segment (start 161.034375 92.991876) (end 156.628124 92.991876) (width 0.2) (layer "F.Cu") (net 8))
 (segment (start 156.628124 92.991876) (end 147.639624 101.980376) (width 0.2) (layer "F.Cu") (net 8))
 (segment (start 141.981875 112.401875) (end 142.01 112.43) (width 0.2) (layer "F.Cu") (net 9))
 (segment (start 141.981875 112.041876) (end 141.981875 112.401875) (width 0.2) (layer "F.Cu") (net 9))
 (segment (start 141.981875 107.760376) (end 133.661875 99.440376) (width 0.2) (layer "B.Cu") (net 9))
 (segment (start 141.981875 112.041876) (end 141.981875 107.760376) (width 0.2) (layer "B.Cu") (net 9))
 (segment (start 145.492499 96.5) (end 134.062251 96.5) (width 0.2) (layer "B.Cu") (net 10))
 (segment (start 161.034375 112.041876) (end 145.492499 96.5) (width 0.2) (layer "B.Cu") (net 10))
 (segment (start 134.062251 96.5) (end 133.661875 96.900376) (width 0.2) (layer "B.Cu") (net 10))
 (segment (start 138.062251 89.96) (end 133.661875 94.360376) (width 0.2) (layer "B.Cu") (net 11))
 (segment (start 174.93 85.8) (end 152.03 85.8) (width 0.2) (layer "B.Cu") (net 11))
 (segment (start 147.87 89.96) (end 138.062251 89.96) (width 0.2) (layer "B.Cu") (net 11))
 (segment (start 180.084375 90.954375) (end 174.93 85.8) (width 0.2) (layer "B.Cu") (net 11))
 (segment (start 152.03 85.8) (end 147.87 89.96) (width 0.2) (layer "B.Cu") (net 11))
 (segment (start 180.084375 112.041876) (end 180.084375 90.954375) (width 0.2) (layer "B.Cu") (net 11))
 (segment (start 116.329624 96.900376) (end 118.421875 96.900376) (width 0.2) (layer "B.Cu") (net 5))
 (segment (start 119.55 109.94) (end 116.15 106.54) (width 0.2) (layer "B.Cu") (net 5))
 (segment (start 116.15 106.54) (end 116.15 97.08) (width 0.2) (layer "B.Cu") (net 5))
 (segment (start 116.15 97.08) (end 116.329624 96.900376) (width 0.2) (layer "B.Cu") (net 5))
 (segment (start 120.35 109.94) (end 119.55 109.94) (width 0.2) (layer "B.Cu") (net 5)))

